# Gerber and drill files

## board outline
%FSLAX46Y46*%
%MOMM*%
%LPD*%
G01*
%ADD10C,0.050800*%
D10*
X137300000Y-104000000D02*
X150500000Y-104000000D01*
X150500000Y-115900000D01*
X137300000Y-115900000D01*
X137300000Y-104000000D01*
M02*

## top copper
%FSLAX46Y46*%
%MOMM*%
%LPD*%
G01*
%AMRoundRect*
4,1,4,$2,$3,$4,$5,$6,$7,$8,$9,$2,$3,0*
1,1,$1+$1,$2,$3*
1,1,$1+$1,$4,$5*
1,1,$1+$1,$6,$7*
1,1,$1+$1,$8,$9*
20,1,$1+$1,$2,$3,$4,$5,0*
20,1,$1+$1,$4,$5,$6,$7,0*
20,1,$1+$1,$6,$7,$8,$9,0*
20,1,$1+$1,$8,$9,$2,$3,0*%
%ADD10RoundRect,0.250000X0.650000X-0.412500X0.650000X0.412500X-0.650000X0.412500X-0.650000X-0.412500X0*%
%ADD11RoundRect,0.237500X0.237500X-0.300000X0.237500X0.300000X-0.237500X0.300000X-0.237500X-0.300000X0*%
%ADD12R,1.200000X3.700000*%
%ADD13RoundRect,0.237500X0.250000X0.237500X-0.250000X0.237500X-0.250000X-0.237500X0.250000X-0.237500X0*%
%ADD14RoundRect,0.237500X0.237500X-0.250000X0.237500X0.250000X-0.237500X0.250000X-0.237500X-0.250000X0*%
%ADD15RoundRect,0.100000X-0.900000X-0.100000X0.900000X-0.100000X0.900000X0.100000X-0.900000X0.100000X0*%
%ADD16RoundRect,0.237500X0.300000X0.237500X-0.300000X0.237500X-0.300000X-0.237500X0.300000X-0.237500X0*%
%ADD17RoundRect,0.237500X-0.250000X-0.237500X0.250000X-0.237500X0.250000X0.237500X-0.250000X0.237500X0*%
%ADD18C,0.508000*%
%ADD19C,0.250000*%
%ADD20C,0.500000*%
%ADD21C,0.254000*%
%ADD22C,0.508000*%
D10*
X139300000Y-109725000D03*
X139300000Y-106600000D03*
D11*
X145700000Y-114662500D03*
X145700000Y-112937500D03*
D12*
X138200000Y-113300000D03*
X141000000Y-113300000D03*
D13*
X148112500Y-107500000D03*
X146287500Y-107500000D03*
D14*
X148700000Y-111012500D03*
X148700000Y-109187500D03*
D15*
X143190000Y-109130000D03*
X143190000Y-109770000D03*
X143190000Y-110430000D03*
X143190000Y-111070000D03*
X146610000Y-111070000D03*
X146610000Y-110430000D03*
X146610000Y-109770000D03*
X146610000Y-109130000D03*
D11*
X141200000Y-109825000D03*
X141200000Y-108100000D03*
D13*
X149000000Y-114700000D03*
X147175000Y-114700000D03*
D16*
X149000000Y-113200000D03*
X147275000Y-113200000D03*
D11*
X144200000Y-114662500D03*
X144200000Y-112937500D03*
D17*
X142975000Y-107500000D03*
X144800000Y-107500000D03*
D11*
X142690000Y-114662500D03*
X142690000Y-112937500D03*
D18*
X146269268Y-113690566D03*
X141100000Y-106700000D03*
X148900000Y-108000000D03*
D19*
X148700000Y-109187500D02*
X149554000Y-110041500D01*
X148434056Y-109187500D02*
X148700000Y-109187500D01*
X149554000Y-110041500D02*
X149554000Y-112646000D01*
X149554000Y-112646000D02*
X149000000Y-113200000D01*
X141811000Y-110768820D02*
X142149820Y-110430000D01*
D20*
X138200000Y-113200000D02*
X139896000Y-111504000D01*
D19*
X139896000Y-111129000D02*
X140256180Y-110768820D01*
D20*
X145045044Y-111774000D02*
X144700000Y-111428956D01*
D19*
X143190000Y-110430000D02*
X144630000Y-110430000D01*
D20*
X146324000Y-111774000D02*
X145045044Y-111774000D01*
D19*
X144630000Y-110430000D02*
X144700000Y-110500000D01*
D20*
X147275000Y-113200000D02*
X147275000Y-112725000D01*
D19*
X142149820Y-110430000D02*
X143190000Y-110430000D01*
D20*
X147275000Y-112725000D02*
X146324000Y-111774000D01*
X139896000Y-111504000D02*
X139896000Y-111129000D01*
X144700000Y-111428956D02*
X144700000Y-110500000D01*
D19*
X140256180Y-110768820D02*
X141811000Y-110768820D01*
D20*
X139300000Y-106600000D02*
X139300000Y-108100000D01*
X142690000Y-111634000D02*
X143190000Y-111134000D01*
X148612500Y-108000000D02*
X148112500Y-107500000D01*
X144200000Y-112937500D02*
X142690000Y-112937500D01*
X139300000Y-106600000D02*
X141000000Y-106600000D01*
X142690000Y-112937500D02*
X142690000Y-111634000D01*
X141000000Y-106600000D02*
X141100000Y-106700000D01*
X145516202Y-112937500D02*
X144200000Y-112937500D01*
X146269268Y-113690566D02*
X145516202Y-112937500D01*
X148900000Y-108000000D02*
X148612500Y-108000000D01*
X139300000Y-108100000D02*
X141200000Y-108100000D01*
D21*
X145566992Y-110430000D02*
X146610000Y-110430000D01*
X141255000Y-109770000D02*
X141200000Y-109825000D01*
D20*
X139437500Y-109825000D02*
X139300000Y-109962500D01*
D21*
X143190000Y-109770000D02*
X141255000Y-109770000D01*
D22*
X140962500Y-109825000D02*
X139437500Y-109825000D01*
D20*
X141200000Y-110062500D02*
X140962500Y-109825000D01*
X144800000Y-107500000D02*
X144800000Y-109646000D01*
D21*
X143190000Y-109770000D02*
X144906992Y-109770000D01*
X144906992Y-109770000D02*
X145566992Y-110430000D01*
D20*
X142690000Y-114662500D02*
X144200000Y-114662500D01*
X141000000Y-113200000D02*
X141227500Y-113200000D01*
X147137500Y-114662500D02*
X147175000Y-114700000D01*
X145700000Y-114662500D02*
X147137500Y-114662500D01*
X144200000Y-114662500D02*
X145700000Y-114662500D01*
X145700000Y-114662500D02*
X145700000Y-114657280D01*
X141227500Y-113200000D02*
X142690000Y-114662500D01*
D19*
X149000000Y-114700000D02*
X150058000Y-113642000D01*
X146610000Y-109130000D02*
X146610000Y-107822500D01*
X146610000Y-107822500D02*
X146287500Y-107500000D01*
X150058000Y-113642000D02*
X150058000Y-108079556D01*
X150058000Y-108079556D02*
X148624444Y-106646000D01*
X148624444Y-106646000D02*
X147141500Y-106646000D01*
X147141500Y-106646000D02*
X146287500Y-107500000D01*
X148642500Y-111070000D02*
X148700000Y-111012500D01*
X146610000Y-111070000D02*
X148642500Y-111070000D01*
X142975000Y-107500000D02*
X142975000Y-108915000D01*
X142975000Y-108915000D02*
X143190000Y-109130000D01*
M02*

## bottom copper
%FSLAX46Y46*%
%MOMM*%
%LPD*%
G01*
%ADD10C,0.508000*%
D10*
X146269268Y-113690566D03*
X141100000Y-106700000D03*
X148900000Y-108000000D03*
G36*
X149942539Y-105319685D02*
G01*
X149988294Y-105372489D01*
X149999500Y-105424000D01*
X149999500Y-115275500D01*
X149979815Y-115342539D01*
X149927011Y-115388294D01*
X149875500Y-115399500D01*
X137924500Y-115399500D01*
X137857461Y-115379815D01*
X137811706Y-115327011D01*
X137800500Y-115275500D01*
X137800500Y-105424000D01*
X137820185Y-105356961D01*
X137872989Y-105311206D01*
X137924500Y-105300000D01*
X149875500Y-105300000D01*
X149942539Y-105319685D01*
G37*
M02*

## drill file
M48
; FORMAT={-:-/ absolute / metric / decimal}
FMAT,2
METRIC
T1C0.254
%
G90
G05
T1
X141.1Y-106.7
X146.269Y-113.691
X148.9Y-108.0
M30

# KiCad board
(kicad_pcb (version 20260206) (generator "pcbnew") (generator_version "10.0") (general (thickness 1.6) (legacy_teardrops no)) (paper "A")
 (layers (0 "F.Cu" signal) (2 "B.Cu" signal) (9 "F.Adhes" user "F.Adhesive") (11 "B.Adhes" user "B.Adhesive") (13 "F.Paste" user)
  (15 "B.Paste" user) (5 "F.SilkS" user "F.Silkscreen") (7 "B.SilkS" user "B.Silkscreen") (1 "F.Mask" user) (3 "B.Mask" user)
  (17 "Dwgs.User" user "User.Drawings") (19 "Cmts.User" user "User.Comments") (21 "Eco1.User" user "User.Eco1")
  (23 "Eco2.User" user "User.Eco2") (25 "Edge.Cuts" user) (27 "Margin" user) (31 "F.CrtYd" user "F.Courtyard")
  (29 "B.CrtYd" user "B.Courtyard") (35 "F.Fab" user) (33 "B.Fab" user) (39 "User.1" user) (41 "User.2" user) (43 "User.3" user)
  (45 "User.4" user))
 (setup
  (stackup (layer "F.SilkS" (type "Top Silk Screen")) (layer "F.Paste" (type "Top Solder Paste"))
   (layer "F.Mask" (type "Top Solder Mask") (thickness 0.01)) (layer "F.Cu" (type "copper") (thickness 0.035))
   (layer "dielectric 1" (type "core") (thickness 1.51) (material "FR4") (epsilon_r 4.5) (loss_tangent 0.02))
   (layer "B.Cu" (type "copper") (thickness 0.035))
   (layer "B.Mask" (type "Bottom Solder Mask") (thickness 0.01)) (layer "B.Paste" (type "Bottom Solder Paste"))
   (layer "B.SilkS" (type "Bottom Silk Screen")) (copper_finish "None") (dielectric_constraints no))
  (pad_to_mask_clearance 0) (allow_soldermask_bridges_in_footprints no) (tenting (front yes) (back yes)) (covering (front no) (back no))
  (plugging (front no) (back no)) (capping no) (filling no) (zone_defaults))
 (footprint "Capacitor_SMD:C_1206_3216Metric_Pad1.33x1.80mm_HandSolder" (layer "F.Cu") (at 139.3 108.1625 90)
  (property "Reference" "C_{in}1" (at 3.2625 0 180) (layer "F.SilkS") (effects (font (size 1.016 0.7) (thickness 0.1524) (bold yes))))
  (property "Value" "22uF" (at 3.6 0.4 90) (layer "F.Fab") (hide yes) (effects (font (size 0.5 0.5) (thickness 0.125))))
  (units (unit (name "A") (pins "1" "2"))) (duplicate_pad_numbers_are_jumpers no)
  (pad "1" smd roundrect (at -1.5625 0 90) (size 1.325 1.8) (layers "F.Cu" "F.Mask" "F.Paste") (roundrect_rratio 0.188679) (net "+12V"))
  (pad "2" smd roundrect (at 1.5625 0 90) (size 1.325 1.8) (layers "F.Cu" "F.Mask" "F.Paste") (roundrect_rratio 0.188679) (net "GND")))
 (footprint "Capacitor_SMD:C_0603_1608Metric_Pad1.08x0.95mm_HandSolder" (layer "F.Cu") (at 145.7 113.8 90)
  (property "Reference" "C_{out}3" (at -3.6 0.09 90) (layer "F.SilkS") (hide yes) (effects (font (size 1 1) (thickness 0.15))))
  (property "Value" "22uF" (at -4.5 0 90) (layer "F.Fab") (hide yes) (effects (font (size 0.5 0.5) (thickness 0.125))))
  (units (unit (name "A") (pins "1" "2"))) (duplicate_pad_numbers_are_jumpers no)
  (pad "1" smd roundrect (at -0.8625 0 90) (size 1.075 0.95) (layers "F.Cu" "F.Mask" "F.Paste") (roundrect_rratio 0.25) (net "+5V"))
  (pad "2" smd roundrect (at 0.8625 0 90) (size 1.075 0.95) (layers "F.Cu" "F.Mask" "F.Paste") (roundrect_rratio 0.25) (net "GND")))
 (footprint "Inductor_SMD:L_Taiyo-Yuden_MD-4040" (layer "F.Cu") (at 139.6 113.3)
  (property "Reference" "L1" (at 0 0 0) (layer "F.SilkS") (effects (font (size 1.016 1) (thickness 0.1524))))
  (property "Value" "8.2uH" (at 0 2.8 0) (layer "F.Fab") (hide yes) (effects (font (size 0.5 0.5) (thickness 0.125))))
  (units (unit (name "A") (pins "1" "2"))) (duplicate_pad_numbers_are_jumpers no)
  (pad "1" smd rect (at -1.4 0) (size 1.2 3.7) (layers "F.Cu" "F.Mask" "F.Paste") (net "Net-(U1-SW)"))
  (pad "2" smd rect (at 1.4 0) (size 1.2 3.7) (layers "F.Cu" "F.Mask" "F.Paste") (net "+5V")))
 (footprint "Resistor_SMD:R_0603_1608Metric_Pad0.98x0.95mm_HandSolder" (layer "F.Cu") (at 147.2 107.5 180)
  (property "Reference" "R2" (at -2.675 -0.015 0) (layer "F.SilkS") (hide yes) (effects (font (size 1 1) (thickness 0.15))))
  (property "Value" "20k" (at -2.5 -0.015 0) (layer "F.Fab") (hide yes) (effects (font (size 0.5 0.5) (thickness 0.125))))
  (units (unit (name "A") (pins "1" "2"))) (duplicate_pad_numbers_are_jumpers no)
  (pad "1" smd roundrect (at -0.9125 0 180) (size 0.975 0.95) (layers "F.Cu" "F.Mask" "F.Paste") (roundrect_rratio 0.25) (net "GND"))
  (pad "2" smd roundrect (at 0.9125 0 180) (size 0.975 0.95) (layers "F.Cu" "F.Mask" "F.Paste") (roundrect_rratio 0.25) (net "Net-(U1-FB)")))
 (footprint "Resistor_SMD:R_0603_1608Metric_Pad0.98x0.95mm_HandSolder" (layer "F.Cu") (at 148.7 110.1 90)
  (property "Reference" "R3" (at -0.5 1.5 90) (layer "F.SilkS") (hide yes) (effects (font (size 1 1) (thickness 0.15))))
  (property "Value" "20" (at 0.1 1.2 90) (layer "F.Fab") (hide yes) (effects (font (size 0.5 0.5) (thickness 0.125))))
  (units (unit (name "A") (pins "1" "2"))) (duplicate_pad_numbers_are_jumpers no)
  (pad "1" smd roundrect (at -0.9125 0 90) (size 0.975 0.95) (layers "F.Cu" "F.Mask" "F.Paste") (roundrect_rratio 0.25)
   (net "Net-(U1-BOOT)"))
  (pad "2" smd roundrect (at 0.9125 0 90) (size 0.975 0.95) (layers "F.Cu" "F.Mask" "F.Paste") (roundrect_rratio 0.25)
   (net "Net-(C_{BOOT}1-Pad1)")))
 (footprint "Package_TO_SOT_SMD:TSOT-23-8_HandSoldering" (layer "F.Cu") (at 144.9 110.1)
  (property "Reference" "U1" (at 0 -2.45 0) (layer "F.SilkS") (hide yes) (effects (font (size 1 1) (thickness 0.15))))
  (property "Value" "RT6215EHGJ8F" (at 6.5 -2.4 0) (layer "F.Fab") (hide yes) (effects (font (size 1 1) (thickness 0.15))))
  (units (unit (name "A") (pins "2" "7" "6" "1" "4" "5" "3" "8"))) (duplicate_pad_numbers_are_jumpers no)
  (pad "1" smd roundrect (at -1.71 -0.97) (size 2 0.4) (layers "F.Cu" "F.Mask" "F.Paste") (roundrect_rratio 0.25) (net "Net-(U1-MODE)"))
  (pad "2" smd roundrect (at -1.71 -0.33) (size 2 0.4) (layers "F.Cu" "F.Mask" "F.Paste") (roundrect_rratio 0.25) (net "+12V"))
  (pad "3" smd roundrect (at -1.71 0.33) (size 2 0.4) (layers "F.Cu" "F.Mask" "F.Paste") (roundrect_rratio 0.25) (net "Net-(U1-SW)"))
  (pad "4" smd roundrect (at -1.71 0.97) (size 2 0.4) (layers "F.Cu" "F.Mask" "F.Paste") (roundrect_rratio 0.25) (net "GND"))
  (pad "5" smd roundrect (at 1.71 0.97) (size 2 0.4) (layers "F.Cu" "F.Mask" "F.Paste") (roundrect_rratio 0.25) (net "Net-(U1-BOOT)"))
  (pad "6" smd roundrect (at 1.71 0.33) (size 2 0.4) (layers "F.Cu" "F.Mask" "F.Paste") (roundrect_rratio 0.25) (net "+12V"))
  (pad "7" smd roundrect (at 1.71 -0.33) (size 2 0.4) (layers "F.Cu" "F.Mask" "F.Paste") (roundrect_rratio 0.25)
   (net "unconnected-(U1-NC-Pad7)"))
  (pad "8" smd roundrect (at 1.71 -0.97) (size 2 0.4) (layers "F.Cu" "F.Mask" "F.Paste") (roundrect_rratio 0.25) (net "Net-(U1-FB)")))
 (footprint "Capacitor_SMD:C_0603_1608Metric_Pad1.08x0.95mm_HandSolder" (layer "F.Cu") (at 141.2 108.9625 90)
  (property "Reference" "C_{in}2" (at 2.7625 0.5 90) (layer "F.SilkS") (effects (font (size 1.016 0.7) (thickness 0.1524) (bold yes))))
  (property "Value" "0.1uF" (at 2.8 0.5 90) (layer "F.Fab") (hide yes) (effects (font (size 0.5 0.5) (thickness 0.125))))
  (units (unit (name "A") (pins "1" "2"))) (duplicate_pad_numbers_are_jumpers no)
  (pad "1" smd roundrect (at -0.8625 0 90) (size 1.075 0.95) (layers "F.Cu" "F.Mask" "F.Paste") (roundrect_rratio 0.25) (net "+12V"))
  (pad "2" smd roundrect (at 0.8625 0 90) (size 1.075 0.95) (layers "F.Cu" "F.Mask" "F.Paste") (roundrect_rratio 0.25) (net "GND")))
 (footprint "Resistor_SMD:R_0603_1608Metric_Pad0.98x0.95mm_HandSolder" (layer "F.Cu") (at 148.0875 114.7 180)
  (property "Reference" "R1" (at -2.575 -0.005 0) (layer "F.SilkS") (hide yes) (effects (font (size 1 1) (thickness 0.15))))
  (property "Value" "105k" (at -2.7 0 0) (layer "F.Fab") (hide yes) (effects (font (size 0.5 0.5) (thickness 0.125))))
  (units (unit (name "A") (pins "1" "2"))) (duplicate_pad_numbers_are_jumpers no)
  (pad "1" smd roundrect (at -0.9125 0 180) (size 0.975 0.95) (layers "F.Cu" "F.Mask" "F.Paste") (roundrect_rratio 0.25) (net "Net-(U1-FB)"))
  (pad "2" smd roundrect (at 0.9125 0 180) (size 0.975 0.95) (layers "F.Cu" "F.Mask" "F.Paste") (roundrect_rratio 0.25) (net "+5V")))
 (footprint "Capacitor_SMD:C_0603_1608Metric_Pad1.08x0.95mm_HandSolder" (layer "F.Cu") (at 148.1375 113.2 180)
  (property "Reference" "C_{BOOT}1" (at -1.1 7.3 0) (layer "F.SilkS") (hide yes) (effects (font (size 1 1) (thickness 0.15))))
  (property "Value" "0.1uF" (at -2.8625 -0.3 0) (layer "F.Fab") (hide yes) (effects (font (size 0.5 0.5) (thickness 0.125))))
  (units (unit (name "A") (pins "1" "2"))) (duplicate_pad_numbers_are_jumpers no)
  (pad "1" smd roundrect (at -0.8625 0 180) (size 1.075 0.95) (layers "F.Cu" "F.Mask" "F.Paste") (roundrect_rratio 0.25)
   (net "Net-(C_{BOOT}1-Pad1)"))
  (pad "2" smd roundrect (at 0.8625 0 180) (size 1.075 0.95) (layers "F.Cu" "F.Mask" "F.Paste") (roundrect_rratio 0.25) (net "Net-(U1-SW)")))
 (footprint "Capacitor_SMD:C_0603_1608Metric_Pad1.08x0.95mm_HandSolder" (layer "F.Cu") (at 144.2 113.8 90)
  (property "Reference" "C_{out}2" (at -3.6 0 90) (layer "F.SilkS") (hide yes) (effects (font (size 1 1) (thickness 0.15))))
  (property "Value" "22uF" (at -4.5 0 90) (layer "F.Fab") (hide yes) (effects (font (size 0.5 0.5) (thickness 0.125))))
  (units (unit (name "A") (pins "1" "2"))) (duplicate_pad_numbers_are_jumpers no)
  (pad "1" smd roundrect (at -0.8625 0 90) (size 1.075 0.95) (layers "F.Cu" "F.Mask" "F.Paste") (roundrect_rratio 0.25) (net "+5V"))
  (pad "2" smd roundrect (at 0.8625 0 90) (size 1.075 0.95) (layers "F.Cu" "F.Mask" "F.Paste") (roundrect_rratio 0.25) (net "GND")))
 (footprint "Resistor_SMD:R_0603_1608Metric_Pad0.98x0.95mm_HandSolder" (layer "F.Cu") (at 143.8875 107.5)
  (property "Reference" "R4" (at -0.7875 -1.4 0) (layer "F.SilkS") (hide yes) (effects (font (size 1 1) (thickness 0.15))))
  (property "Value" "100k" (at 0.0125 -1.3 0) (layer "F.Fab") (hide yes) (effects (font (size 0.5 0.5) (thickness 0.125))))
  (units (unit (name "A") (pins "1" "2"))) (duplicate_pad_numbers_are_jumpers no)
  (pad "1" smd roundrect (at -0.9125 0) (size 0.975 0.95) (layers "F.Cu" "F.Mask" "F.Paste") (roundrect_rratio 0.25) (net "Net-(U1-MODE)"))
  (pad "2" smd roundrect (at 0.9125 0) (size 0.975 0.95) (layers "F.Cu" "F.Mask" "F.Paste") (roundrect_rratio 0.25) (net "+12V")))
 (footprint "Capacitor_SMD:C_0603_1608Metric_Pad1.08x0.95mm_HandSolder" (layer "F.Cu") (at 142.69 113.8 90)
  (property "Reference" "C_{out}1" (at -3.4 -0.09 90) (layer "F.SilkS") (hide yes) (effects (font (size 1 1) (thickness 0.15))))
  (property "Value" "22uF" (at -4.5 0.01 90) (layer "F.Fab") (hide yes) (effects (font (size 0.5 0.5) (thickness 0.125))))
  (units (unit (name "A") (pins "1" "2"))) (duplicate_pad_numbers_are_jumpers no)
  (pad "1" smd roundrect (at -0.8625 0 90) (size 1.075 0.95) (layers "F.Cu" "F.Mask" "F.Paste") (roundrect_rratio 0.25) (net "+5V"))
  (pad "2" smd roundrect (at 0.8625 0 90) (size 1.075 0.95) (layers "F.Cu" "F.Mask" "F.Paste") (roundrect_rratio 0.25) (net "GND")))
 (gr_rect (start 137.3 104) (end 150.5 115.9) (stroke (width 0.0508) (type default)) (fill no) (layer "Edge.Cuts"))
 (segment (start 148.7 109.1875) (end 149.554 110.0415) (width 0.25) (layer "F.Cu") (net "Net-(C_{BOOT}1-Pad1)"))
 (segment (start 148.434056 109.1875) (end 148.7 109.1875) (width 0.25) (layer "F.Cu") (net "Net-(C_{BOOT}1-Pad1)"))
 (segment (start 149.554 110.0415) (end 149.554 112.646) (width 0.25) (layer "F.Cu") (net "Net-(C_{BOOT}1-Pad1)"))
 (segment (start 149.554 112.646) (end 149 113.2) (width 0.25) (layer "F.Cu") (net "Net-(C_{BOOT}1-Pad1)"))
 (segment (start 141.811 110.76882) (end 142.14982 110.43) (width 0.25) (layer "F.Cu") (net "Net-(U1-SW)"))
 (segment (start 138.2 113.2) (end 139.896 111.504) (width 0.5) (layer "F.Cu") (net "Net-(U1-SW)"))
 (segment (start 139.896 111.129) (end 140.25618 110.76882) (width 0.25) (layer "F.Cu") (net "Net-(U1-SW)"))
 (segment (start 145.045044 111.774) (end 144.7 111.428956) (width 0.5) (layer "F.Cu") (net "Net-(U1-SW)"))
 (segment (start 143.19 110.43) (end 144.63 110.43) (width 0.25) (layer "F.Cu") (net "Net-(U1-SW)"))
 (segment (start 146.324 111.774) (end 145.045044 111.774) (width 0.5) (layer "F.Cu") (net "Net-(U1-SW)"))
 (segment (start 144.63 110.43) (end 144.7 110.5) (width 0.25) (layer "F.Cu") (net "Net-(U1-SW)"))
 (segment (start 147.275 113.2) (end 147.275 112.725) (width 0.5) (layer "F.Cu") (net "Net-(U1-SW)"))
 (segment (start 142.14982 110.43) (end 143.19 110.43) (width 0.25) (layer "F.Cu") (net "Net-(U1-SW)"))
 (segment (start 147.275 112.725) (end 146.324 111.774) (width 0.5) (layer "F.Cu") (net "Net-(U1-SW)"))
 (segment (start 139.896 111.504) (end 139.896 111.129) (width 0.5) (layer "F.Cu") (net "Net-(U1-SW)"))
 (segment (start 144.7 111.428956) (end 144.7 110.5) (width 0.5) (layer "F.Cu") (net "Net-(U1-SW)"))
 (segment (start 140.25618 110.76882) (end 141.811 110.76882) (width 0.25) (layer "F.Cu") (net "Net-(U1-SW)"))
 (segment (start 139.3 106.6) (end 139.3 108.1) (width 0.5) (layer "F.Cu") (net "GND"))
 (segment (start 142.69 111.634) (end 143.19 111.134) (width 0.5) (layer "F.Cu") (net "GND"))
 (segment (start 148.6125 108) (end 148.1125 107.5) (width 0.5) (layer "F.Cu") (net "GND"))
 (segment (start 144.2 112.9375) (end 142.69 112.9375) (width 0.5) (layer "F.Cu") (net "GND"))
 (segment (start 139.3 106.6) (end 141 106.6) (width 0.5) (layer "F.Cu") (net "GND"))
 (segment (start 142.69 112.9375) (end 142.69 111.634) (width 0.5) (layer "F.Cu") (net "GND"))
 (segment (start 141 106.6) (end 141.1 106.7) (width 0.5) (layer "F.Cu") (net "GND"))
 (segment (start 145.516202 112.9375) (end 144.2 112.9375) (width 0.5) (layer "F.Cu") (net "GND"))
 (segment (start 146.269268 113.690566) (end 145.516202 112.9375) (width 0.5) (layer "F.Cu") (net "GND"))
 (segment (start 148.9 108) (end 148.6125 108) (width 0.5) (layer "F.Cu") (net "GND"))
 (segment (start 139.3 108.1) (end 141.2 108.1) (width 0.5) (layer "F.Cu") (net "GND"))
 (via (at 146.269268 113.690566) (size 0.508) (drill 0.254) (layers "F.Cu" "B.Cu") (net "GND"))
 (via (at 141.1 106.7) (size 0.508) (drill 0.254) (layers "F.Cu" "B.Cu") (free yes) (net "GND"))
 (via (at 148.9 108) (size 0.508) (drill 0.254) (layers "F.Cu" "B.Cu") (free yes) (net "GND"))
 (segment (start 145.566992 110.43) (end 146.61 110.43) (width 0.254) (layer "F.Cu") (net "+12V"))
 (segment (start 141.255 109.77) (end 141.2 109.825) (width 0.254) (layer "F.Cu") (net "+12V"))
 (segment (start 139.4375 109.825) (end 139.3 109.9625) (width 0.5) (layer "F.Cu") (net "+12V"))
 (segment (start 143.19 109.77) (end 141.255 109.77) (width 0.254) (layer "F.Cu") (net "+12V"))
 (segment (start 140.9625 109.825) (end 139.4375 109.825) (width 0.508) (layer "F.Cu") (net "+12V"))
 (segment (start 141.2 110.0625) (end 140.9625 109.825) (width 0.5) (layer "F.Cu") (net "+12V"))
 (segment (start 144.8 107.5) (end 144.8 109.646) (width 0.5) (layer "F.Cu") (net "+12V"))
 (segment (start 143.19 109.77) (end 144.906992 109.77) (width 0.254) (layer "F.Cu") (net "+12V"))
 (segment (start 144.906992 109.77) (end 145.566992 110.43) (width 0.254) (layer "F.Cu") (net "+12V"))
 (segment (start 142.69 114.6625) (end 144.2 114.6625) (width 0.5) (layer "F.Cu") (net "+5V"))
 (segment (start 141 113.2) (end 141.2275 113.2) (width 0.5) (layer "F.Cu") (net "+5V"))
 (segment (start 147.1375 114.6625) (end 147.175 114.7) (width 0.5) (layer "F.Cu") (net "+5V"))
 (segment (start 145.7 114.6625) (end 147.1375 114.6625) (width 0.5) (layer "F.Cu") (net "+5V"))
 (segment (start 144.2 114.6625) (end 145.7 114.6625) (width 0.5) (layer "F.Cu") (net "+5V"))
 (segment (start 145.7 114.6625) (end 145.7 114.65728) (width 0.5) (layer "F.Cu") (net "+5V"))
 (segment (start 141.2275 113.2) (end 142.69 114.6625) (width 0.5) (layer "F.Cu") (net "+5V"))
 (segment (start 149 114.7) (end 150.058 113.642) (width 0.25) (layer "F.Cu") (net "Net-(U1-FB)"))
 (segment (start 146.61 109.13) (end 146.61 107.8225) (width 0.25) (layer "F.Cu") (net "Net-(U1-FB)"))
 (segment (start 146.61 107.8225) (end 146.2875 107.5) (width 0.25) (layer "F.Cu") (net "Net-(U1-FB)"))
 (segment (start 150.058 113.642) (end 150.058 108.079556) (width 0.25) (layer "F.Cu") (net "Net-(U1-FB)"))
 (segment (start 150.058 108.079556) (end 148.624444 106.646) (width 0.25) (layer "F.Cu") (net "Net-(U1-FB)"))
 (segment (start 148.624444 106.646) (end 147.1415 106.646) (width 0.25) (layer "F.Cu") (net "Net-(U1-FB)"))
 (segment (start 147.1415 106.646) (end 146.2875 107.5) (width 0.25) (layer "F.Cu") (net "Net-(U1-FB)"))
 (segment (start 148.6425 111.07) (end 148.7 111.0125) (width 0.25) (layer "F.Cu") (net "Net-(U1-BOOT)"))
 (segment (start 146.61 111.07) (end 148.6425 111.07) (width 0.25) (layer "F.Cu") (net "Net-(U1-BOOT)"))
 (segment (start 142.975 107.5) (end 142.975 108.915) (width 0.25) (layer "F.Cu") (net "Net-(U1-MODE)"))
 (segment (start 142.975 108.915) (end 143.19 109.13) (width 0.25) (layer "F.Cu") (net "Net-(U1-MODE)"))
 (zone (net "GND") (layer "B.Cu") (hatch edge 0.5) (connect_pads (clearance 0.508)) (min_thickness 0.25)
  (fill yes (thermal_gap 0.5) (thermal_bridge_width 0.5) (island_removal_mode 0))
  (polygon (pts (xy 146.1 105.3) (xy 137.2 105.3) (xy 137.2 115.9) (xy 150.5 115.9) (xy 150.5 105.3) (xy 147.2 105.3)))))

